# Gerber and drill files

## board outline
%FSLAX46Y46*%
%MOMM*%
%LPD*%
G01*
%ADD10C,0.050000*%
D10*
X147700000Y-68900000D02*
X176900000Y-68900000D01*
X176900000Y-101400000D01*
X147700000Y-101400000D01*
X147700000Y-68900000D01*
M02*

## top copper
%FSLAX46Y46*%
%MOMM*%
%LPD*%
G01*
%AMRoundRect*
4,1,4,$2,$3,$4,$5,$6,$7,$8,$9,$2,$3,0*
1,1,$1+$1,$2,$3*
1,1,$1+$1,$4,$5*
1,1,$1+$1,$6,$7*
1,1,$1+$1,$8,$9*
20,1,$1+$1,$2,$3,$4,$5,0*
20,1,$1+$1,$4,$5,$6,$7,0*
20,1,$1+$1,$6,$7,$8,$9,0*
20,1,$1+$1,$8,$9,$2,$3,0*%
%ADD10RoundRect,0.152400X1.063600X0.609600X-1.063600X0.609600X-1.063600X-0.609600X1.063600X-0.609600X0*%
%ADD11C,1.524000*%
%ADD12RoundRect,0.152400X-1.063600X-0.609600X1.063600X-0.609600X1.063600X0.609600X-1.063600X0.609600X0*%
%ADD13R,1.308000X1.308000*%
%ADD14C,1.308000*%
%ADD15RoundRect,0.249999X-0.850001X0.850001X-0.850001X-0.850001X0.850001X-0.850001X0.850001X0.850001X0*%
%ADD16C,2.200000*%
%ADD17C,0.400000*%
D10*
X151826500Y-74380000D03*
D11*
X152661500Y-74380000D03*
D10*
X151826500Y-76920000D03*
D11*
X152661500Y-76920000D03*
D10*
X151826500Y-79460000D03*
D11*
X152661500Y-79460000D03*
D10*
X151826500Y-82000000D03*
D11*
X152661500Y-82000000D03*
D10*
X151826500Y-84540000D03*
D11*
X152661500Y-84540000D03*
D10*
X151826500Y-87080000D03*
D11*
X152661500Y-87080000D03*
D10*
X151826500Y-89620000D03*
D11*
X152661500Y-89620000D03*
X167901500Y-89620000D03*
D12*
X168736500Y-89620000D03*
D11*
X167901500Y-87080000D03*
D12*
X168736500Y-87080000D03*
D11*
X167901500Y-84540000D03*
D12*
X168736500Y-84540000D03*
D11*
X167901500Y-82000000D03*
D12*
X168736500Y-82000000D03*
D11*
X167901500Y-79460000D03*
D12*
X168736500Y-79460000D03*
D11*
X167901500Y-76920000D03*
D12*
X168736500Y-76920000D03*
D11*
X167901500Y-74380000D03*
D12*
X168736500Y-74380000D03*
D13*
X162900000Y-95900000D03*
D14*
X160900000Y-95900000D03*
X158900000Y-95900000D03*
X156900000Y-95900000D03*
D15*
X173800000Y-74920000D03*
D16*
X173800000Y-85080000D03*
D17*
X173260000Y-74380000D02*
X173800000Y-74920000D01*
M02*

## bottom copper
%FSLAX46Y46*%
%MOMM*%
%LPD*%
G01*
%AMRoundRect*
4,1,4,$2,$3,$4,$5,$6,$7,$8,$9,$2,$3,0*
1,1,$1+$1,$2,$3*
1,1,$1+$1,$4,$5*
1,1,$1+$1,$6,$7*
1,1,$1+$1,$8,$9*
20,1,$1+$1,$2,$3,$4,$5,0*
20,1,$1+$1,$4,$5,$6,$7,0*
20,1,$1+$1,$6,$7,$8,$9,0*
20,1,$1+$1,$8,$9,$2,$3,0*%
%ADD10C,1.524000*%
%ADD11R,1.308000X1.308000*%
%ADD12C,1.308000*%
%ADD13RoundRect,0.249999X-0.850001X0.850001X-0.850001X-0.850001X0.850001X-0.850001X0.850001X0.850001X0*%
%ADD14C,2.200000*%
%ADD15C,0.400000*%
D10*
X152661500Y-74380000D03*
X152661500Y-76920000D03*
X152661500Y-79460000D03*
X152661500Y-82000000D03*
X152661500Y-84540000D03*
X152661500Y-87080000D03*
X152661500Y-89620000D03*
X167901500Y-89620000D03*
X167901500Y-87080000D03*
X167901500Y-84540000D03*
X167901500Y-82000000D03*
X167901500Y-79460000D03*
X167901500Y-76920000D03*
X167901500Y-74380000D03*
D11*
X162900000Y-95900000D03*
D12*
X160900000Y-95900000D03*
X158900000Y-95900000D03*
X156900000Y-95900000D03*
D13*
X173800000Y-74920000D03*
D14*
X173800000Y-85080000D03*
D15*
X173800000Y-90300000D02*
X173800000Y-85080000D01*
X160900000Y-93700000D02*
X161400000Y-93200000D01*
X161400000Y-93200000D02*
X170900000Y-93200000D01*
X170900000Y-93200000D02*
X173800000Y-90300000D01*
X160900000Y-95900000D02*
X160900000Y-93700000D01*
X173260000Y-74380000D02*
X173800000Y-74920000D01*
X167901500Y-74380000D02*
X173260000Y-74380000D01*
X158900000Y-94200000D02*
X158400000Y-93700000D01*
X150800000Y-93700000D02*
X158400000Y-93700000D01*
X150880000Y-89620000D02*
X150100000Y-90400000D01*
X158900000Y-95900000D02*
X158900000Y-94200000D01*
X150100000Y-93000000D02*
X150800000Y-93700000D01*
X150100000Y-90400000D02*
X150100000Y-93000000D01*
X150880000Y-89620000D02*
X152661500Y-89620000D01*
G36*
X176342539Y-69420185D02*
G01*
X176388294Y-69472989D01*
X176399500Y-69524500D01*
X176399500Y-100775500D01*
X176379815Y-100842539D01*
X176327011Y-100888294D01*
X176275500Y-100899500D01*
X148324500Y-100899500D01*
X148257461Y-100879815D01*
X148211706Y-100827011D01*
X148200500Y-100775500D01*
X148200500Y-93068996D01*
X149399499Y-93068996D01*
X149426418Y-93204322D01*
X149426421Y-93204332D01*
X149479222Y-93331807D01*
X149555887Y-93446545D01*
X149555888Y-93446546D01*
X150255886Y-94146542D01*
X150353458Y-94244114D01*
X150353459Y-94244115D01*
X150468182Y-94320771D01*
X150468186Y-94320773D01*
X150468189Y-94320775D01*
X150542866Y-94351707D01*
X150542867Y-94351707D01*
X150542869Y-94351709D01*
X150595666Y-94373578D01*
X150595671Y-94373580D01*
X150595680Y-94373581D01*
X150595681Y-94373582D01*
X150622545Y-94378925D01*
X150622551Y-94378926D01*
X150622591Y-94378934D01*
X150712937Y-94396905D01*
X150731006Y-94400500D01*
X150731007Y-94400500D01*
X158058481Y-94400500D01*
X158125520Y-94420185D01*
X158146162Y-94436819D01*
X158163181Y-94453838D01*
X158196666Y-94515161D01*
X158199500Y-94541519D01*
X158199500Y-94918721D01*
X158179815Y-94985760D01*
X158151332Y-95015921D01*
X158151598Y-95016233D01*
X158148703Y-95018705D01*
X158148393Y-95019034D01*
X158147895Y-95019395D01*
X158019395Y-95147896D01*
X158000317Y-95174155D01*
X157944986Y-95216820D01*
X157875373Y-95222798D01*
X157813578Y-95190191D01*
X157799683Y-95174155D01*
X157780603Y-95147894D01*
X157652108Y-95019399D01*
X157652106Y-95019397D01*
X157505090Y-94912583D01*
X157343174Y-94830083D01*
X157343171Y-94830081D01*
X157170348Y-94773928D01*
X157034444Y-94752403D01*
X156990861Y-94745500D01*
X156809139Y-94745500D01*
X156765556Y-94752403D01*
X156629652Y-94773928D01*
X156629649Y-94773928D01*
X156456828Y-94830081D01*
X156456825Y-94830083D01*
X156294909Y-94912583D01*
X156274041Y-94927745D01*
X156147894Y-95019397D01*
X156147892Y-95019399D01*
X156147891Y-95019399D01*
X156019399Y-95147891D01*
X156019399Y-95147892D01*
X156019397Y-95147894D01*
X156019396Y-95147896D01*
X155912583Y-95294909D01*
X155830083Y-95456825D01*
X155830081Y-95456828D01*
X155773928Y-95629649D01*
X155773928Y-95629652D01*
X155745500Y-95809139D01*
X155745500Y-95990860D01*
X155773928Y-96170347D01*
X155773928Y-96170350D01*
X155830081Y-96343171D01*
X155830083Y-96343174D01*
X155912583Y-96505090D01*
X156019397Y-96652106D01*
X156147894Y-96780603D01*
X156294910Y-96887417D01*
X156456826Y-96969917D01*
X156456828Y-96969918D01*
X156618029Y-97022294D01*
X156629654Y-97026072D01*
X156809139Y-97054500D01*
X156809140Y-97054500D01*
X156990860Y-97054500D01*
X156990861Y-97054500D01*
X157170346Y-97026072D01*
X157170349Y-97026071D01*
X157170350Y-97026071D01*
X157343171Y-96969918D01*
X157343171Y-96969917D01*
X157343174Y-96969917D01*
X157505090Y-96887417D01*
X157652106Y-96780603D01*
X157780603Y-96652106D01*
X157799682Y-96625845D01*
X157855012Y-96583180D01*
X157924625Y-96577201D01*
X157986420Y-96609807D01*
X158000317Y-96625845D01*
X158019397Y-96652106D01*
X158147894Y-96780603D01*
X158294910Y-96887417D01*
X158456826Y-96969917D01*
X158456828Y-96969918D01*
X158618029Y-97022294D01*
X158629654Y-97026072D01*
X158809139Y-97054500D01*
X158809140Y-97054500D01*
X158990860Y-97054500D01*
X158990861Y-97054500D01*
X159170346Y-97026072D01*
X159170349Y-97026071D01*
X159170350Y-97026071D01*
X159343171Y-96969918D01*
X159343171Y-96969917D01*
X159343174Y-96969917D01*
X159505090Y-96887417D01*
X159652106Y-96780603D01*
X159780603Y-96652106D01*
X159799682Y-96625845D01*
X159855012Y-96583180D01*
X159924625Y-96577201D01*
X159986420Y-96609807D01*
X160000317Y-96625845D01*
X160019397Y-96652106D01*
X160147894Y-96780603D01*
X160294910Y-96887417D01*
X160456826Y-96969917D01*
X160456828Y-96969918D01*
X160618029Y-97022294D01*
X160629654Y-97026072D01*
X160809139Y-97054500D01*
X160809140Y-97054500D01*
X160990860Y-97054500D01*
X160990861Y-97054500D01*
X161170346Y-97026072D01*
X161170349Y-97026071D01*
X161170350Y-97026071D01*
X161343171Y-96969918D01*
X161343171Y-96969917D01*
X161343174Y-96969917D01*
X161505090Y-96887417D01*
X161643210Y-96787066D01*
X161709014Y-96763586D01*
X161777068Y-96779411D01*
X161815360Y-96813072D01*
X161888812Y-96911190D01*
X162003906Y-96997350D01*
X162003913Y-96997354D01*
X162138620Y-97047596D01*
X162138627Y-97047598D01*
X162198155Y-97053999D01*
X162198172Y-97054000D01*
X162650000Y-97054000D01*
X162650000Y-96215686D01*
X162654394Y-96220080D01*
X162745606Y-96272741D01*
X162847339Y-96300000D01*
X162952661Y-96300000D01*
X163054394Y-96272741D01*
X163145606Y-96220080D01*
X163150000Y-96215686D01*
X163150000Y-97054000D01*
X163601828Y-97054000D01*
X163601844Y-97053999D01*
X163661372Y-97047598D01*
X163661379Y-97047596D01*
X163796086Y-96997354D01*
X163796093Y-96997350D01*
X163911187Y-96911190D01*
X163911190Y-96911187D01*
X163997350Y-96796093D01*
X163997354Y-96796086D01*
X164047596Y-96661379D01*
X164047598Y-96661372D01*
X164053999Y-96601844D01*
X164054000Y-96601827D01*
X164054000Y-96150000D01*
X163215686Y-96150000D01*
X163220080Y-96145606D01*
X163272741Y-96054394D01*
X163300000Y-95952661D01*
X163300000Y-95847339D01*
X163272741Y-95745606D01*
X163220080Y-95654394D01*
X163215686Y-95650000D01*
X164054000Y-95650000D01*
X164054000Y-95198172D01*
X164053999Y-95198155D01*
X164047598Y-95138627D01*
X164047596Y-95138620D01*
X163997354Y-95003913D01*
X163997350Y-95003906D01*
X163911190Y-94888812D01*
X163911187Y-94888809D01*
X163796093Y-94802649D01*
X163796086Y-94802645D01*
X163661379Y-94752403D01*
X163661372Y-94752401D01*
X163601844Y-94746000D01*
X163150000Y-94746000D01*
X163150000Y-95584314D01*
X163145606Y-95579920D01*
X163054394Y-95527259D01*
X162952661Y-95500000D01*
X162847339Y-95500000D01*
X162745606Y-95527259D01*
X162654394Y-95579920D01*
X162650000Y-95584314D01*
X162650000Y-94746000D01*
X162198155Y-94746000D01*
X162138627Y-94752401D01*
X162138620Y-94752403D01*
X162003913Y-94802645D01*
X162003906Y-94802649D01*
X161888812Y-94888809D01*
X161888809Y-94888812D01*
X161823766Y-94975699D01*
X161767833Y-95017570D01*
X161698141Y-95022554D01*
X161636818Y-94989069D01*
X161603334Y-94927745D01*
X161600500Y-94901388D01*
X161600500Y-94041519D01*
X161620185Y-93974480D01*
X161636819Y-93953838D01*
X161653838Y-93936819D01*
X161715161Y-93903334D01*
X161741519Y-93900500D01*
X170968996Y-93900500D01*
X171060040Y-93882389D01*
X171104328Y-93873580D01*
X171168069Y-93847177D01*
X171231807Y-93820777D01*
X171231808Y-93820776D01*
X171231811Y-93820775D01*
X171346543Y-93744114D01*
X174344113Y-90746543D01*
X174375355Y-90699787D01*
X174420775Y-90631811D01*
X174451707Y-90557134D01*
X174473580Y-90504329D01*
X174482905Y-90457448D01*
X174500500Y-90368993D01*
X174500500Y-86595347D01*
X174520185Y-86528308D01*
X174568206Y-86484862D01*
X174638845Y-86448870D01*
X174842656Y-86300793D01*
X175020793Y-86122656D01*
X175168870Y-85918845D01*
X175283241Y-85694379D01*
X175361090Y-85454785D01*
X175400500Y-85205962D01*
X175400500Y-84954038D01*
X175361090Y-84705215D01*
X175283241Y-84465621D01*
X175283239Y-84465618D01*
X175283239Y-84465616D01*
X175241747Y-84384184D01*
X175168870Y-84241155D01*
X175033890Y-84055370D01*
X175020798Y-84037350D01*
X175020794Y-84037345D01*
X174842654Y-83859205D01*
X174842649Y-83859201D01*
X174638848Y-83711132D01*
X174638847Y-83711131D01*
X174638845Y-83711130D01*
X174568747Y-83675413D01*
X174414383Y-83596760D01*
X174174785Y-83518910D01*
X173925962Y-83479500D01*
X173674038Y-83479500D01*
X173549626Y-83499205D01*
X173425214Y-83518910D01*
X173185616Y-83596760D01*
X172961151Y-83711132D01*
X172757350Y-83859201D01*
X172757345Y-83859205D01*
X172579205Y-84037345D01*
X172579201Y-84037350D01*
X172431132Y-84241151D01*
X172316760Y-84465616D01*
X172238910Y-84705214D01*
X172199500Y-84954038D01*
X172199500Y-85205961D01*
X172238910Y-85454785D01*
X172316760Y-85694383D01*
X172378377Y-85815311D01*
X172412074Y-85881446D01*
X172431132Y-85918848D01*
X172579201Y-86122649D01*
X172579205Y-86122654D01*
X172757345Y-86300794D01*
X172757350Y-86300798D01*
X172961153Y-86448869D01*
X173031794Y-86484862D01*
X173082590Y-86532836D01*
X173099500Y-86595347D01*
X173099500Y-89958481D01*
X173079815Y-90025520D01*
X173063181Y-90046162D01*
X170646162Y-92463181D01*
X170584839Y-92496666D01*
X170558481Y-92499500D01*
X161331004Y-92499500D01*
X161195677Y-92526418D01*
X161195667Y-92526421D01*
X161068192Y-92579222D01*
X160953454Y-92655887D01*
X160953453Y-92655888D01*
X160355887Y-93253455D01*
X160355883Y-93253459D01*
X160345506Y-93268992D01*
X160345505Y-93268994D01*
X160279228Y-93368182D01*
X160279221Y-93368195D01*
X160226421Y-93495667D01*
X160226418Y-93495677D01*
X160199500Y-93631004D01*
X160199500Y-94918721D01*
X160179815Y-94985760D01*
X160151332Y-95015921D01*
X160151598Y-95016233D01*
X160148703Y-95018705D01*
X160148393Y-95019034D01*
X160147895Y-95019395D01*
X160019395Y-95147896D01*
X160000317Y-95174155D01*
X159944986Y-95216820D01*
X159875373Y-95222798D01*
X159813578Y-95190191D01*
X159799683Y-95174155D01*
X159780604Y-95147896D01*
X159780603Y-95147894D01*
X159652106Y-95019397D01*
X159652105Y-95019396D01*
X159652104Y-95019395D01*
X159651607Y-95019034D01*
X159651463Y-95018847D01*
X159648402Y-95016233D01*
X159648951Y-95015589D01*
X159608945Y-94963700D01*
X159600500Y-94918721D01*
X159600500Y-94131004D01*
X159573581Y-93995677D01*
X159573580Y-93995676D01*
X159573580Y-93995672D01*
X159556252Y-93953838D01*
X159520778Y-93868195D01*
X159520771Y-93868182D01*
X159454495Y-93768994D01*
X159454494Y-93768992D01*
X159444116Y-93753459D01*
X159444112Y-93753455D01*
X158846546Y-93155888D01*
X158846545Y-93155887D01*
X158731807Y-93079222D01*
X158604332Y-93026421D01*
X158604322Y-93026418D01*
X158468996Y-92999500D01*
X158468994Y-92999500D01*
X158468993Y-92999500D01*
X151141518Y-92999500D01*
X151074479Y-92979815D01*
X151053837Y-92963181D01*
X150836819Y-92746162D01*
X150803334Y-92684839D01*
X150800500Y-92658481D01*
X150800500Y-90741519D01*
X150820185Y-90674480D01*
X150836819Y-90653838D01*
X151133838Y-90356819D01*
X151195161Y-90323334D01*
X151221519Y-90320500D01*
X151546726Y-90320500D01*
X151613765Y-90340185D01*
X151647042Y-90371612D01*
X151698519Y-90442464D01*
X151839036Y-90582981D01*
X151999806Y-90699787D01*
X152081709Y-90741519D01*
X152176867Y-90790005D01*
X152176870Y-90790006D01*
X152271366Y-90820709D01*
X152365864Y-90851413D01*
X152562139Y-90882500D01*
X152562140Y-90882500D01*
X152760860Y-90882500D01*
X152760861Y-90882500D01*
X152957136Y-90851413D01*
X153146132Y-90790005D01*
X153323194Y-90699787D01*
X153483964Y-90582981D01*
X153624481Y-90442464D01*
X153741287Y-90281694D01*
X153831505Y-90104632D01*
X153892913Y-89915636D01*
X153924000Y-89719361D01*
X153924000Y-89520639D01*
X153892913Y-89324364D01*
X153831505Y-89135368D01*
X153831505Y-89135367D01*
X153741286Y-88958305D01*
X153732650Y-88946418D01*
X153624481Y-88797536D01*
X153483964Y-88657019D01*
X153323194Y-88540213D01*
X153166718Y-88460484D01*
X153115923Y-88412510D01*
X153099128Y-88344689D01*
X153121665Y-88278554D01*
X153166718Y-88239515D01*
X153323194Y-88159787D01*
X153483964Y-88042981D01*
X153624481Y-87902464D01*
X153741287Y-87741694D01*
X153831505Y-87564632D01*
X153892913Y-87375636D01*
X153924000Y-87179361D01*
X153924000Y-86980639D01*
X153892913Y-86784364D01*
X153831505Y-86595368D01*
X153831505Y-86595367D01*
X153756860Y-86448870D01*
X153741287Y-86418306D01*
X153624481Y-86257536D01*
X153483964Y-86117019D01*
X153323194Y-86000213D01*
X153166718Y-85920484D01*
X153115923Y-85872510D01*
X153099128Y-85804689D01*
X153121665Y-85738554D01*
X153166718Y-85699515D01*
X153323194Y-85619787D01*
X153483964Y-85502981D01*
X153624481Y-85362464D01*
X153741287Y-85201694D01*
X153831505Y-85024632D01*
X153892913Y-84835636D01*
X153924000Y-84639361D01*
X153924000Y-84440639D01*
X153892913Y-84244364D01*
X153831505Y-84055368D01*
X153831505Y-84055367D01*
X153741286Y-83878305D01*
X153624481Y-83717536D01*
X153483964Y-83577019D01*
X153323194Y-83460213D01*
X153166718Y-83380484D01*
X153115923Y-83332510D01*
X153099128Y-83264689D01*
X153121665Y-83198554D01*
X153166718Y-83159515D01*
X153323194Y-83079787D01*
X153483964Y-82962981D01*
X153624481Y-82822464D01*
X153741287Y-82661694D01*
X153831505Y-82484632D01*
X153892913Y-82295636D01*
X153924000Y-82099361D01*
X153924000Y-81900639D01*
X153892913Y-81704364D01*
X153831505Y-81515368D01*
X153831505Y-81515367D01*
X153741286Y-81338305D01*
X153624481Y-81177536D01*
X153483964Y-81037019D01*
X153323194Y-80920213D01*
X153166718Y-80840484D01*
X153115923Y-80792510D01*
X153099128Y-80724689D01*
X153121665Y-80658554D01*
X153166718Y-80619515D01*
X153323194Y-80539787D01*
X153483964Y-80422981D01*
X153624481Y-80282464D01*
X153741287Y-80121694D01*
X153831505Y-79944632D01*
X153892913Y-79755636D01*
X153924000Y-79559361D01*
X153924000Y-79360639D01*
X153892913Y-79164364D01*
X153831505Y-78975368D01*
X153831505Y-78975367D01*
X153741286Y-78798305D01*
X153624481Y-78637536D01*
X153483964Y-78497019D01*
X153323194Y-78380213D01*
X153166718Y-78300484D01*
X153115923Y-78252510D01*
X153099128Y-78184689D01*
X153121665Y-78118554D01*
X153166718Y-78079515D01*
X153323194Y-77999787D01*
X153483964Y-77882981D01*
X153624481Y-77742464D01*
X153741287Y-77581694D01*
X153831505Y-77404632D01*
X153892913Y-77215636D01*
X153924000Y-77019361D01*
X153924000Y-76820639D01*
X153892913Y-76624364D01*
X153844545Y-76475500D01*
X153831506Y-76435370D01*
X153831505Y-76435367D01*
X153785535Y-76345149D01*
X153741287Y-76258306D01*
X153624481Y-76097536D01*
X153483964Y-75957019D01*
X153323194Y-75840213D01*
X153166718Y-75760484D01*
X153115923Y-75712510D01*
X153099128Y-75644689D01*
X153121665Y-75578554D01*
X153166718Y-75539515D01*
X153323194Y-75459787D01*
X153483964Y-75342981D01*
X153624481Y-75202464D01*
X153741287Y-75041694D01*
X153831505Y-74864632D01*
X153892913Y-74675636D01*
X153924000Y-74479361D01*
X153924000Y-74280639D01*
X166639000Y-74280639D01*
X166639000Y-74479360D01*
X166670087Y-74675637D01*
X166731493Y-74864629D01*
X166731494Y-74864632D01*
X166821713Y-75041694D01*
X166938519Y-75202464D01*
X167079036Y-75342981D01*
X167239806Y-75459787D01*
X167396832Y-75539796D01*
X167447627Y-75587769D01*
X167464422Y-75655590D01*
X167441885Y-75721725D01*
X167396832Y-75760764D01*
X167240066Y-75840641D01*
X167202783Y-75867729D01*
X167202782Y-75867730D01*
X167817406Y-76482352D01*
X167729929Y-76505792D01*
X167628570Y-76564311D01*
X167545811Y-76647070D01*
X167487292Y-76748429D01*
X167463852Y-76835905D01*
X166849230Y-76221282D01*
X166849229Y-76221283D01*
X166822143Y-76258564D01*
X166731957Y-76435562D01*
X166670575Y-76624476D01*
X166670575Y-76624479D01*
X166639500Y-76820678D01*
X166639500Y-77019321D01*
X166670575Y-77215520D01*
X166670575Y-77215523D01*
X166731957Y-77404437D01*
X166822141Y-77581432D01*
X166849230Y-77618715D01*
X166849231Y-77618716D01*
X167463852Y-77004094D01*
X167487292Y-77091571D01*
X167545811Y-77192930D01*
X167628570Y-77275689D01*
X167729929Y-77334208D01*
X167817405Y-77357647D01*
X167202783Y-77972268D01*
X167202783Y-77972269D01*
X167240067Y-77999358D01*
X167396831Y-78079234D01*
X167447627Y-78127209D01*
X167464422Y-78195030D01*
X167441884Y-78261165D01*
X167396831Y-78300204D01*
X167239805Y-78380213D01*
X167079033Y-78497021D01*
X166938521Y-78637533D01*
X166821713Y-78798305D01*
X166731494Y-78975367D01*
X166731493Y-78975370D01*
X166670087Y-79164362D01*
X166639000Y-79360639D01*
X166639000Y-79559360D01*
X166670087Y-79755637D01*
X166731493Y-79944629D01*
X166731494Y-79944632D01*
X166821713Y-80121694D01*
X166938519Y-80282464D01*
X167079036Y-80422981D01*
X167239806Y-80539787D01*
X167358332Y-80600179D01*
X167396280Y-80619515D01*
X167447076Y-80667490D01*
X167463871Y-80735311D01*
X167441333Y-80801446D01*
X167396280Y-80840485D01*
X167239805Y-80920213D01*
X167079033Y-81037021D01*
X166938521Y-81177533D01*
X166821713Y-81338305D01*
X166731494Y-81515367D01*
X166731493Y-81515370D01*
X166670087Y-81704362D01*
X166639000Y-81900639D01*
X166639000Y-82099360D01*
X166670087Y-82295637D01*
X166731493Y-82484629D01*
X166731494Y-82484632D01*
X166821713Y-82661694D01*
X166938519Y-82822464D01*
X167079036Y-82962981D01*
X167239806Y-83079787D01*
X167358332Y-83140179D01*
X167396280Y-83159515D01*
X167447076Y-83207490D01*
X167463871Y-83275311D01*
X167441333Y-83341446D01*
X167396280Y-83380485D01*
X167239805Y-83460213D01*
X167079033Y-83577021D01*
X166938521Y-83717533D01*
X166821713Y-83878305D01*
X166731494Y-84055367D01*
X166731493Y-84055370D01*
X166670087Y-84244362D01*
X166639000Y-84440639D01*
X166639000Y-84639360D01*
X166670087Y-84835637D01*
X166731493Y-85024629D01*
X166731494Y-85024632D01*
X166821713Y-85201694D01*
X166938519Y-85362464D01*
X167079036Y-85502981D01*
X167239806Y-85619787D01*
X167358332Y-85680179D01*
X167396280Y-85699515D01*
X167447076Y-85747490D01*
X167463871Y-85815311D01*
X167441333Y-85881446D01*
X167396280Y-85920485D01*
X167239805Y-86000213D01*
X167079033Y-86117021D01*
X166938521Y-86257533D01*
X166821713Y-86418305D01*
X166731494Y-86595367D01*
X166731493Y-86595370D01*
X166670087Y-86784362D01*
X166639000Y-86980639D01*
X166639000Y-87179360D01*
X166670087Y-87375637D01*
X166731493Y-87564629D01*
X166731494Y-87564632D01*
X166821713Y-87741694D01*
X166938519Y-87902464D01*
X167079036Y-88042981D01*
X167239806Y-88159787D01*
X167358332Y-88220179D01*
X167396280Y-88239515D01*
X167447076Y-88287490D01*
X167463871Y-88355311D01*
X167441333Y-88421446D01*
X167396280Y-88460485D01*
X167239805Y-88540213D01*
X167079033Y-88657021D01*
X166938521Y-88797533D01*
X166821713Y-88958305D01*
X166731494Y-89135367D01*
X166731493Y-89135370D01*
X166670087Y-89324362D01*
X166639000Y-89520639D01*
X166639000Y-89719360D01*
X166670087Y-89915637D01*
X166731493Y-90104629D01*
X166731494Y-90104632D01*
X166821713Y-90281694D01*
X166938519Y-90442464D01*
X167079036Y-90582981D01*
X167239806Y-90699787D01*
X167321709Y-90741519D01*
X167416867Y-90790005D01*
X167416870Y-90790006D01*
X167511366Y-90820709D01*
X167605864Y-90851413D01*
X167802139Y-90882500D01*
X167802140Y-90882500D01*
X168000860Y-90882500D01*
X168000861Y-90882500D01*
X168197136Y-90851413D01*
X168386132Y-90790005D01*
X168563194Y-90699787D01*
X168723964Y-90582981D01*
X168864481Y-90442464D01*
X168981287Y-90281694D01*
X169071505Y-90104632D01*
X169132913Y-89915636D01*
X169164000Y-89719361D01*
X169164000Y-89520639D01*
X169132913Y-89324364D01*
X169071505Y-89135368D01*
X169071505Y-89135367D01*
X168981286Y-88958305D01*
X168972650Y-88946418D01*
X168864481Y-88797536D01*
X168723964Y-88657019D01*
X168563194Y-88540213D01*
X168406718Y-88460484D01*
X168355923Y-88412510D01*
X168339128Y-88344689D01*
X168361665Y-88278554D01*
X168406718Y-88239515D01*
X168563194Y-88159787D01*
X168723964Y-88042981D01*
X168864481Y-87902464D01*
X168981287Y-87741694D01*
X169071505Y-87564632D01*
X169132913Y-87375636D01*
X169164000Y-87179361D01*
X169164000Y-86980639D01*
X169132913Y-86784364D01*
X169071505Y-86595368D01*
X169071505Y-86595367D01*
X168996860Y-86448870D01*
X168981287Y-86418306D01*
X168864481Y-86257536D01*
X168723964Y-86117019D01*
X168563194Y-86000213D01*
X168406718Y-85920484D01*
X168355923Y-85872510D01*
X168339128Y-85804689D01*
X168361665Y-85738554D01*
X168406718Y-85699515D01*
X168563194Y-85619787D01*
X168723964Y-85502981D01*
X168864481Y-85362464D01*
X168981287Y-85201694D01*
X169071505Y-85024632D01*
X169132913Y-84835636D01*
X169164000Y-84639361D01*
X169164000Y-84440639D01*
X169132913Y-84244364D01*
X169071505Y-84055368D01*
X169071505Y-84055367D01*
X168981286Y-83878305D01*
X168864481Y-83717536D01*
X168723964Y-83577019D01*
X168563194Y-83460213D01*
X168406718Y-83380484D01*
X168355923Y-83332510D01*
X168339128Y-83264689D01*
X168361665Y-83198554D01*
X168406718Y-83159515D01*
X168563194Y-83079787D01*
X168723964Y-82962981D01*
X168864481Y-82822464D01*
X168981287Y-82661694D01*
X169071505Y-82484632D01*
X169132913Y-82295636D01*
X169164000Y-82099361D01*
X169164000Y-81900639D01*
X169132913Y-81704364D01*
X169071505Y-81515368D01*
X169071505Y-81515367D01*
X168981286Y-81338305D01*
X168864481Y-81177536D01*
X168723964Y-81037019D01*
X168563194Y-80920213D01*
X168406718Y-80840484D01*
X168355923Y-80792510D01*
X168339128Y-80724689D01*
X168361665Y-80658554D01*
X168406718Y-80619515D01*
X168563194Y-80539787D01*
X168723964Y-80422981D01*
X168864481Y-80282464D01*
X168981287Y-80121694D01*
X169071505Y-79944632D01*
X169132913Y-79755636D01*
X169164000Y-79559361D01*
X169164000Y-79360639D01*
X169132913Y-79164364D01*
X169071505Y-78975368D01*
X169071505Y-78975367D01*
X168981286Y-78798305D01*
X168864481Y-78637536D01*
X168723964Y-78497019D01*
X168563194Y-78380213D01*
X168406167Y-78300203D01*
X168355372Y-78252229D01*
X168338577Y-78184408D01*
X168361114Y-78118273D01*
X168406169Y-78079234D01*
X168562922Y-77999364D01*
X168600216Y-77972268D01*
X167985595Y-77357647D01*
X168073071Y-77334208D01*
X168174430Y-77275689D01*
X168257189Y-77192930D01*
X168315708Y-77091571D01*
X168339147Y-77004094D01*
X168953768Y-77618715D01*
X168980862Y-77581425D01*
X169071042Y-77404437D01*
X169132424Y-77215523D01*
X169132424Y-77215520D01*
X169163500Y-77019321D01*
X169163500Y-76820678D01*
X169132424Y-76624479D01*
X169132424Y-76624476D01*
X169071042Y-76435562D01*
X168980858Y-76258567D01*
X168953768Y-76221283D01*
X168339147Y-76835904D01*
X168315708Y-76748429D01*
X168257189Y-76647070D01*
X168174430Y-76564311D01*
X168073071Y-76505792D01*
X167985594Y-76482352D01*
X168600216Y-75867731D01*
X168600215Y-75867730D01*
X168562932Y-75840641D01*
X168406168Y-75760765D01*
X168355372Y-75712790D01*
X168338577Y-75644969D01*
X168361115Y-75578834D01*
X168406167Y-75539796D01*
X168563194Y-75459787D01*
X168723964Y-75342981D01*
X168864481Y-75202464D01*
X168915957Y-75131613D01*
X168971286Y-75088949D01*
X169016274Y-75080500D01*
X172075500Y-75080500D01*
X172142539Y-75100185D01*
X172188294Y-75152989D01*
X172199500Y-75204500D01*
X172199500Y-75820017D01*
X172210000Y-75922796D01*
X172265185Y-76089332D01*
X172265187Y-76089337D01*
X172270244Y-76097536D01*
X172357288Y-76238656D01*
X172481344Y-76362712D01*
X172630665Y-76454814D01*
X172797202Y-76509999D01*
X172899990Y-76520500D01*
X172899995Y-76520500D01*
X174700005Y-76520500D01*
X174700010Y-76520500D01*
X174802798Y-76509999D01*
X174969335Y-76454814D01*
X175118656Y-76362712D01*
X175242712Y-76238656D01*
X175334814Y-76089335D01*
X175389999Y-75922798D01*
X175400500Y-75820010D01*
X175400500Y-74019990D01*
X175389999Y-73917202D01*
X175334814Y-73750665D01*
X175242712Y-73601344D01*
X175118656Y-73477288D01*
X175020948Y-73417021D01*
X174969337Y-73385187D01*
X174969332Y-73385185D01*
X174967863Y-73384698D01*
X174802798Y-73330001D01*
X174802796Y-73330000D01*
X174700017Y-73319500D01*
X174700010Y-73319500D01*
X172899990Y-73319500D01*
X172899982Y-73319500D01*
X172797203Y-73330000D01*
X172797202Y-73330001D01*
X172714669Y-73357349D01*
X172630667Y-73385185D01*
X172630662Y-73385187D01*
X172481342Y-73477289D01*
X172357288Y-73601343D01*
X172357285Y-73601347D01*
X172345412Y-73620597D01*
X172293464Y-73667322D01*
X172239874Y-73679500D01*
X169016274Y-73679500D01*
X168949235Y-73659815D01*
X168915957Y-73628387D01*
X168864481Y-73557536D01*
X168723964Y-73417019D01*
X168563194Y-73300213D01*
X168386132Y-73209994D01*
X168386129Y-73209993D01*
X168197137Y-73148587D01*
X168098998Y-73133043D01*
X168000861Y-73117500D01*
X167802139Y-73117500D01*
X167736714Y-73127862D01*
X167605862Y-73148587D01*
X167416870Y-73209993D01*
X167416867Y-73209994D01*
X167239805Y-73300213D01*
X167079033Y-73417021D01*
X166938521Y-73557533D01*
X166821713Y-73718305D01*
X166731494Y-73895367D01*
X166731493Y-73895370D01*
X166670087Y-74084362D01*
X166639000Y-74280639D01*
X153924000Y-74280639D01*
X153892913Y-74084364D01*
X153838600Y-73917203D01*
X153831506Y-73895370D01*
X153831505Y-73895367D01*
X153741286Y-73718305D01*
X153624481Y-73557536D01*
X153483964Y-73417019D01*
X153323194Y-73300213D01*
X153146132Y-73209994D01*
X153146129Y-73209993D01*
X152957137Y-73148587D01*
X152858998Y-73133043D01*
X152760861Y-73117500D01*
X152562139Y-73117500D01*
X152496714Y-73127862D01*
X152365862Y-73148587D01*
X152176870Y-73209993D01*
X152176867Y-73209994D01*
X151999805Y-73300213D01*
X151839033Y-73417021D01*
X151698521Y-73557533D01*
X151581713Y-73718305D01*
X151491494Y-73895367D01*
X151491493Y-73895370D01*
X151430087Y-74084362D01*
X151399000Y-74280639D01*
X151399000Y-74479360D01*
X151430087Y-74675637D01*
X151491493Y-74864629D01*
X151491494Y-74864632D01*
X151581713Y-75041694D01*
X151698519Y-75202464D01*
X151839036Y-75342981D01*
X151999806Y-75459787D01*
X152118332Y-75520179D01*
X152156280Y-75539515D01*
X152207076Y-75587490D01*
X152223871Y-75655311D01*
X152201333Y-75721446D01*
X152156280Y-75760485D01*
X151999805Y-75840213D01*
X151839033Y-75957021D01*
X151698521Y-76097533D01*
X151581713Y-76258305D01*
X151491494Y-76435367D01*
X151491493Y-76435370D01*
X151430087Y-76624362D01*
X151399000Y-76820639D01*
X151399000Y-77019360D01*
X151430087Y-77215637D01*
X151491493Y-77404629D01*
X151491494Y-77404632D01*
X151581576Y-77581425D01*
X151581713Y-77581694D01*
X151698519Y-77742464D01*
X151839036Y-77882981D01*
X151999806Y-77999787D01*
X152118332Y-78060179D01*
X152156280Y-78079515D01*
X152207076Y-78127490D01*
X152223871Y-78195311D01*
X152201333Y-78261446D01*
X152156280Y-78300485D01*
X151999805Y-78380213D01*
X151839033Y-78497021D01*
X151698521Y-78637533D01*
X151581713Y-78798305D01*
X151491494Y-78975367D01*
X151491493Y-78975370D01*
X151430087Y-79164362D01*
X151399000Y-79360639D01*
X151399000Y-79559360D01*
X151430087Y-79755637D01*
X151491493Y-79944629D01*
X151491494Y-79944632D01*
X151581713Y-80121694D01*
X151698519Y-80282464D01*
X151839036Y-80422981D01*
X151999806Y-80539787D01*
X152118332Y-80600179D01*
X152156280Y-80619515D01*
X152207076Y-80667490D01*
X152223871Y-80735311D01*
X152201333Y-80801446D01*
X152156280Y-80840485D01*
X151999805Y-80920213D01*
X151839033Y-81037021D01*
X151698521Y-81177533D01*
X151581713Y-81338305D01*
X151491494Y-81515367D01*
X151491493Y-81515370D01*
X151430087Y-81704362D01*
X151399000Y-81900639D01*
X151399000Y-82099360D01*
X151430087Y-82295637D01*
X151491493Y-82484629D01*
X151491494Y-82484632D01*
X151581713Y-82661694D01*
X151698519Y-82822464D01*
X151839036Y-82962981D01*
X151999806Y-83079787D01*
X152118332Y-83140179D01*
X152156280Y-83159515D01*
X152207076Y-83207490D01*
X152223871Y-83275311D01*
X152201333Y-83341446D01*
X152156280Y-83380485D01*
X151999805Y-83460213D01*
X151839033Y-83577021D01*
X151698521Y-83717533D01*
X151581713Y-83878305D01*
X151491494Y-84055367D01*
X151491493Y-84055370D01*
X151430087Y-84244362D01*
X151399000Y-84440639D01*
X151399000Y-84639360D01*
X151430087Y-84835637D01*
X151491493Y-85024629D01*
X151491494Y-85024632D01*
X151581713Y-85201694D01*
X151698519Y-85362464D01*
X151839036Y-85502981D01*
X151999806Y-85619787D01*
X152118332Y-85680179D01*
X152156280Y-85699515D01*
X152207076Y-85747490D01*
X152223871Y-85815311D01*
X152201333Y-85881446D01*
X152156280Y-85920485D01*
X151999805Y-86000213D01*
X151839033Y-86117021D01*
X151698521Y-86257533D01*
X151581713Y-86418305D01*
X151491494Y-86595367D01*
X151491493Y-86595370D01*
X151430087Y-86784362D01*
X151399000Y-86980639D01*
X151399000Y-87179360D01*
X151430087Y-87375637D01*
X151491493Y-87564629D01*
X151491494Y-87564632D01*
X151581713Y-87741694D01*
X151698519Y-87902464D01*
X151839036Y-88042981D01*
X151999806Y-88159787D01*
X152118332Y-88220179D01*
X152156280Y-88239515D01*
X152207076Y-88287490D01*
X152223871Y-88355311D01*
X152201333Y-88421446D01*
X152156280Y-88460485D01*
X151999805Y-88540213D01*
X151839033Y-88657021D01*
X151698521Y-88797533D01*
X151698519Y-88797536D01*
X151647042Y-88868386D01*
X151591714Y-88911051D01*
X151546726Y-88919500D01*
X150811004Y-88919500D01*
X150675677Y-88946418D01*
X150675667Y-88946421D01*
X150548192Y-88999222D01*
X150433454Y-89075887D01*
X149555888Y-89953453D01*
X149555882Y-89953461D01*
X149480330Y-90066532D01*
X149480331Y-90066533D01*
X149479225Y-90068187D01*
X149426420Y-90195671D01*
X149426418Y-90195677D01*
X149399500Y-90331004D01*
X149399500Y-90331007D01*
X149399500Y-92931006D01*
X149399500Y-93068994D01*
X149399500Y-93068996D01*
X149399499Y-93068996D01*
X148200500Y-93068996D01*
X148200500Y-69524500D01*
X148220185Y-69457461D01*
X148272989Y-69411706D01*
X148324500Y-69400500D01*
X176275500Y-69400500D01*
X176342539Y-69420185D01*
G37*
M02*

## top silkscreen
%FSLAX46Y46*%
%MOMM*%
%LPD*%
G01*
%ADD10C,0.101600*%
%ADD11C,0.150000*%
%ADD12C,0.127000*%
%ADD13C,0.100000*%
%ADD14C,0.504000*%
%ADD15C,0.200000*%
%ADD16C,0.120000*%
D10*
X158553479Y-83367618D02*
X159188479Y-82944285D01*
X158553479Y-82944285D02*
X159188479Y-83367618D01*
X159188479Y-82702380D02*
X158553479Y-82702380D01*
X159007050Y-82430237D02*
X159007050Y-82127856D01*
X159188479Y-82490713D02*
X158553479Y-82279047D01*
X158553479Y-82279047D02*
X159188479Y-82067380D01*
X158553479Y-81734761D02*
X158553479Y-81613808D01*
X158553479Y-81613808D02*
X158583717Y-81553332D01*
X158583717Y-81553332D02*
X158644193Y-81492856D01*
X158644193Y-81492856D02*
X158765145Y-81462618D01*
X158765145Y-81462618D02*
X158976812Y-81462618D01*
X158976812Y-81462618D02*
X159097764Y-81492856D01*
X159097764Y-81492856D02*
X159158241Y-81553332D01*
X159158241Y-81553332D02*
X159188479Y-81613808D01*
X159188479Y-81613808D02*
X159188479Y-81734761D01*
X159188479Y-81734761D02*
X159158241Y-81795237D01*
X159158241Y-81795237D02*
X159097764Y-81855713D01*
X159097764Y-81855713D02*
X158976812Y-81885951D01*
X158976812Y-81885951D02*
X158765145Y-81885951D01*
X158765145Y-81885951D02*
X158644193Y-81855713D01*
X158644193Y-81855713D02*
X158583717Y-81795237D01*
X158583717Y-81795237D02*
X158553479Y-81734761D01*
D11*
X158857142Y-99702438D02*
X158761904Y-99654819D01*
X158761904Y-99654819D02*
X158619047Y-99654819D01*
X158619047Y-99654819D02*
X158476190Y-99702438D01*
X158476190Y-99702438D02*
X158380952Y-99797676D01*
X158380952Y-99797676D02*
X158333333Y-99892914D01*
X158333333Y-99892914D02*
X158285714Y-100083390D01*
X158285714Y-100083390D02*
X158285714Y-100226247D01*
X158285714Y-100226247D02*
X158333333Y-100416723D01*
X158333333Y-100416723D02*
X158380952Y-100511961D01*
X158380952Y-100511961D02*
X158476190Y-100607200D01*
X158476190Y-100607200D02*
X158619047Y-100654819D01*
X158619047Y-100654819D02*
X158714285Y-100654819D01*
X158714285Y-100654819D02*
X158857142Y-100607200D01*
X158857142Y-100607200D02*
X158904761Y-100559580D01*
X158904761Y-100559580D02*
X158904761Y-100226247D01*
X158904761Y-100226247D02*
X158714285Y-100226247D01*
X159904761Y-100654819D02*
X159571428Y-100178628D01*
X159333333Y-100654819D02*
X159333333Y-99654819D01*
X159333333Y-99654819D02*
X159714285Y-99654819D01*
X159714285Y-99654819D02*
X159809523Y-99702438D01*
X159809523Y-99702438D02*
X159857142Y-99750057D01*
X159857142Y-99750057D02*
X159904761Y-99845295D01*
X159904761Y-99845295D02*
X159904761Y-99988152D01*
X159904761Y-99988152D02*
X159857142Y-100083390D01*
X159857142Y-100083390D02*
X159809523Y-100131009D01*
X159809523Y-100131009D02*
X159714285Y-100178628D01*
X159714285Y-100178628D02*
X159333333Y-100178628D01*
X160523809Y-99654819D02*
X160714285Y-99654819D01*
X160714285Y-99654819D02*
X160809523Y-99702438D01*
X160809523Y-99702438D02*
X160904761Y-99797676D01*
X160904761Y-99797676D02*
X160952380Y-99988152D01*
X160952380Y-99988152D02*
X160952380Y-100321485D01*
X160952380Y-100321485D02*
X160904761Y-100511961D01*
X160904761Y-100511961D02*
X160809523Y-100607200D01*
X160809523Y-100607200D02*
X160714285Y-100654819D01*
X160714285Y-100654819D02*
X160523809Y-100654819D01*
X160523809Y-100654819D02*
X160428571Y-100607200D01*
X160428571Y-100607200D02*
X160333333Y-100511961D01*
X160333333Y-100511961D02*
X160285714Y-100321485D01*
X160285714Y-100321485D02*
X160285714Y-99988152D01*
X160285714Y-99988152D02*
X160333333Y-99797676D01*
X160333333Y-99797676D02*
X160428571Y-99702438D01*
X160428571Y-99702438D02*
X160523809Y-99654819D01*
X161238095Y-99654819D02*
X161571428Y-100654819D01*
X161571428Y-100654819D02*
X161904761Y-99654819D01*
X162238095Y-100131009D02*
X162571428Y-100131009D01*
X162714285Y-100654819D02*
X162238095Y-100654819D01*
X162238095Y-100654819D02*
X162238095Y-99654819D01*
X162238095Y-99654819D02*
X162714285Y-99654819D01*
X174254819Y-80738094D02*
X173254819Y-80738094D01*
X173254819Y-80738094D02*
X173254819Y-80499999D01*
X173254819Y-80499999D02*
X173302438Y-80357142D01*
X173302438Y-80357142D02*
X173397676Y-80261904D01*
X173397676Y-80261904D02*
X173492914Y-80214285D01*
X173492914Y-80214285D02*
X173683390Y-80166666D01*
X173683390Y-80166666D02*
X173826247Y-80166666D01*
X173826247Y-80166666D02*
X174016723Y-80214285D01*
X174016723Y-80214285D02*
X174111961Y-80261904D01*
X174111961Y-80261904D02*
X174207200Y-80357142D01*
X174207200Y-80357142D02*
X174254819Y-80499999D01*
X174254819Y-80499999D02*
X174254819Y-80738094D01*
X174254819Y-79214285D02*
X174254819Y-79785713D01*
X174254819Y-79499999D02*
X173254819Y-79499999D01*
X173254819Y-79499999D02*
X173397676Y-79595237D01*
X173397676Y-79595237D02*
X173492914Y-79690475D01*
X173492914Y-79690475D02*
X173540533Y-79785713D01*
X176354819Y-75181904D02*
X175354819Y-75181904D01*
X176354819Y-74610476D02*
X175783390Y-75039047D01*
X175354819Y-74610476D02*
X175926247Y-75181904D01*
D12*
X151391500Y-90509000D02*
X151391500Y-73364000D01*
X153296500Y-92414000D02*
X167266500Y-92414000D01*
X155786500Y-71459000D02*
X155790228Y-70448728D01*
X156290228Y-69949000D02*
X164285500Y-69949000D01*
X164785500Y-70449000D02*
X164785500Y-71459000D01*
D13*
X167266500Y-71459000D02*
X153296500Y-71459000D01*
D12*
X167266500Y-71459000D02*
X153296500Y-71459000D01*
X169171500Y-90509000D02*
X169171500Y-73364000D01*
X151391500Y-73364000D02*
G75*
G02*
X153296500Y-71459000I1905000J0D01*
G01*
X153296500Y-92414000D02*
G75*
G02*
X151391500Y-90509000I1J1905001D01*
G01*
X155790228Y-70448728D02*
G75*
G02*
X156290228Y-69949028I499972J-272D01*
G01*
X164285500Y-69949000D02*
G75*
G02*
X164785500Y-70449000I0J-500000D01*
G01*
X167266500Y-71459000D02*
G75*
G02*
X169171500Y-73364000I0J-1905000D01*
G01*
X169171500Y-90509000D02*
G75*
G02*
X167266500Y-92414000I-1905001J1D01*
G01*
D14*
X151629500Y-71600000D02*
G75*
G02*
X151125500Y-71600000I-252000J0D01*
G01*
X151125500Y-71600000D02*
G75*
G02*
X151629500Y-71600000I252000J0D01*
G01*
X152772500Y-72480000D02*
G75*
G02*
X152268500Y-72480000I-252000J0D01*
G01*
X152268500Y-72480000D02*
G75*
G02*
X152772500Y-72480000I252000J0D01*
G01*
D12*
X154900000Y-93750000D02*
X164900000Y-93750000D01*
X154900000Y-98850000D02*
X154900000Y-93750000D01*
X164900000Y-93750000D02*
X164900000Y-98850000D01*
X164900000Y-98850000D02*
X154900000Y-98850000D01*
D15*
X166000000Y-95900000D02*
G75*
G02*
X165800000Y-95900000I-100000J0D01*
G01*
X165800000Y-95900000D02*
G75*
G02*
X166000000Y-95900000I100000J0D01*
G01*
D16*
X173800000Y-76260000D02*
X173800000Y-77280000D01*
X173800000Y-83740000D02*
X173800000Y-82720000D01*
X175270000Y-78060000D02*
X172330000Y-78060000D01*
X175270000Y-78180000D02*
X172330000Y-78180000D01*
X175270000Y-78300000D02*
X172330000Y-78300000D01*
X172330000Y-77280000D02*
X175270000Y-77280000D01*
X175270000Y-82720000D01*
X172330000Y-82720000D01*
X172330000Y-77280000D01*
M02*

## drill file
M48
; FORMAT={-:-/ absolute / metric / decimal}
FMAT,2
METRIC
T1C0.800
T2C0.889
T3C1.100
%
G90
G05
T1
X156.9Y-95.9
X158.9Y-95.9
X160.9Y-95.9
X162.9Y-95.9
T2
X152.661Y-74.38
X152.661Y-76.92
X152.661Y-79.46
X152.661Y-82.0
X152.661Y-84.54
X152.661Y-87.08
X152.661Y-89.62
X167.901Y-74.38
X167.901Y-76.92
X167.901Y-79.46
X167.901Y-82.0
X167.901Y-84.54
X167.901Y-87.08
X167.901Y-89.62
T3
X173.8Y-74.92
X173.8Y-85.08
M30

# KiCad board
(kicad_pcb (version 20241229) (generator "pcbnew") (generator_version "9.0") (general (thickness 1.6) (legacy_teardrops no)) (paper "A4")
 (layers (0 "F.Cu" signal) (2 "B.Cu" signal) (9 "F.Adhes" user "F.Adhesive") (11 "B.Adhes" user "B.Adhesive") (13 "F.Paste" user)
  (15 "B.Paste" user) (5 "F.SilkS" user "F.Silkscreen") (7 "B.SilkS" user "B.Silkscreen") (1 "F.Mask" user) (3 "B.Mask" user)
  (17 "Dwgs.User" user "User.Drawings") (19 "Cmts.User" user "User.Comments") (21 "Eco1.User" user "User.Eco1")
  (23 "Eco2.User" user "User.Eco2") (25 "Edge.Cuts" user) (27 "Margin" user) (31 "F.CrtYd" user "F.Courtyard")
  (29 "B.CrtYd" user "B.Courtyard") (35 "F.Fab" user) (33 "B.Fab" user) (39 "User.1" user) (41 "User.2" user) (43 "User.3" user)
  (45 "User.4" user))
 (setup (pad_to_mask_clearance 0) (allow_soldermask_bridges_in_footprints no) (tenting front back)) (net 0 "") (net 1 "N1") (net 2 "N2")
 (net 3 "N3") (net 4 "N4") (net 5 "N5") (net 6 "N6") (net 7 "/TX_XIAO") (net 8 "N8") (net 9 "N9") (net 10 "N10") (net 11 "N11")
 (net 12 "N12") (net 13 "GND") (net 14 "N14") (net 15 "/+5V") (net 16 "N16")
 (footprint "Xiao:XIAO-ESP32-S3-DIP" (layer "F.Cu") (at 160.2815 82 90)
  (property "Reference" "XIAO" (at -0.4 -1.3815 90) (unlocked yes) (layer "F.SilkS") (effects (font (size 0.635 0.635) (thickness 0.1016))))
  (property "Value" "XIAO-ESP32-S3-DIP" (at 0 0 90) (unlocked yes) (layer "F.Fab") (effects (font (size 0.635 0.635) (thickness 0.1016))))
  (fp_line (start -8.509 -8.89) (end 8.636 -8.89) (stroke (width 0.127) (type solid)) (layer "F.SilkS"))
  (fp_line (start -10.414 -6.985) (end -10.414 6.985) (stroke (width 0.127) (type solid)) (layer "F.SilkS"))
  (fp_line (start 10.541 -4.495) (end 11.551272 -4.491272) (stroke (width 0.127) (type solid)) (layer "F.SilkS"))
  (fp_line (start 12.051 -3.991272) (end 12.051 4.004) (stroke (width 0.127) (type solid)) (layer "F.SilkS"))
  (fp_line (start 11.551 4.504) (end 10.541 4.504) (stroke (width 0.127) (type solid)) (layer "F.SilkS"))
  (fp_line (start 10.541 6.985) (end 10.541 -6.985) (stroke (width 0.1) (type solid)) (layer "F.SilkS"))
  (fp_line (start 10.541 6.985) (end 10.541 -6.985) (stroke (width 0.127) (type solid)) (layer "F.SilkS"))
  (fp_line (start -8.509 8.89) (end 8.636 8.89) (stroke (width 0.127) (type solid)) (layer "F.SilkS"))
  (fp_arc (start 8.636 -8.89) (mid 9.983038 -8.332038) (end 10.541 -6.985) (stroke (width 0.127) (type solid)) (layer "F.SilkS"))
  (fp_arc (start -10.414 -6.985) (mid -9.856038 -8.332038) (end -8.509 -8.89) (stroke (width 0.127) (type solid)) (layer "F.SilkS"))
  (fp_arc (start 11.551272 -4.491272) (mid 11.904644 -4.344724) (end 12.051 -3.991272) (stroke (width 0.127) (type default))
   (layer "F.SilkS"))
  (fp_arc (start 12.051 4.004) (mid 11.904553 4.357553) (end 11.551 4.504) (stroke (width 0.127) (type default)) (layer "F.SilkS"))
  (fp_arc (start 10.541 6.985) (mid 9.983038 8.332038) (end 8.636 8.89) (stroke (width 0.127) (type solid)) (layer "F.SilkS"))
  (fp_arc (start -8.509 8.89) (mid -9.856038 8.332038) (end -10.414 6.985) (stroke (width 0.127) (type solid)) (layer "F.SilkS"))
  (fp_circle (center 10.4 -8.904) (end 10.654 -8.904) (stroke (width 0.5) (type solid)) (fill yes) (layer "F.SilkS"))
  (fp_circle (center 9.52 -7.761) (end 9.774 -7.761) (stroke (width 0.5) (type solid)) (fill yes) (layer "F.SilkS"))
  (pad "1" smd roundrect (at 7.62 -8.455 180) (size 2.432 1.524) (layers "F.Cu" "F.Mask") (roundrect_rratio 0.1) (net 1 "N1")
   (thermal_bridge_angle 45))
  (pad "1" thru_hole circle (at 7.62 -7.62 180) (size 1.524 1.524) (drill 0.889) (layers "*.Cu" "*.Mask") (remove_unused_layers no)
   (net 1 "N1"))
  (pad "2" smd roundrect (at 5.08 -8.455 180) (size 2.432 1.524) (layers "F.Cu" "F.Mask") (roundrect_rratio 0.1) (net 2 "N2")
   (thermal_bridge_angle 45))
  (pad "2" thru_hole circle (at 5.08 -7.62 180) (size 1.524 1.524) (drill 0.889) (layers "*.Cu" "*.Mask") (remove_unused_layers no)
   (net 2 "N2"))
  (pad "3" smd roundrect (at 2.54 -8.455 180) (size 2.432 1.524) (layers "F.Cu" "F.Mask") (roundrect_rratio 0.1) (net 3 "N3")
   (thermal_bridge_angle 45))
  (pad "3" thru_hole circle (at 2.54 -7.62 180) (size 1.524 1.524) (drill 0.889) (layers "*.Cu" "*.Mask") (remove_unused_layers no)
   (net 3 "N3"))
  (pad "4" smd roundrect (at 0 -8.455 180) (size 2.432 1.524) (layers "F.Cu" "F.Mask") (roundrect_rratio 0.1) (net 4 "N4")
   (thermal_bridge_angle 45))
  (pad "4" thru_hole circle (at 0 -7.62 180) (size 1.524 1.524) (drill 0.889) (layers "*.Cu" "*.Mask") (remove_unused_layers no)
   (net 4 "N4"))
  (pad "5" smd roundrect (at -2.54 -8.455 180) (size 2.432 1.524) (layers "F.Cu" "F.Mask") (roundrect_rratio 0.1) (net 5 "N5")
   (thermal_bridge_angle 45))
  (pad "5" thru_hole circle (at -2.54 -7.62 180) (size 1.524 1.524) (drill 0.889) (layers "*.Cu" "*.Mask") (remove_unused_layers no)
   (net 5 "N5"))
  (pad "6" smd roundrect (at -5.08 -8.455 180) (size 2.432 1.524) (layers "F.Cu" "F.Mask") (roundrect_rratio 0.1) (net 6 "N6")
   (thermal_bridge_angle 45))
  (pad "6" thru_hole circle (at -5.08 -7.62 180) (size 1.524 1.524) (drill 0.889) (layers "*.Cu" "*.Mask") (remove_unused_layers no)
   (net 6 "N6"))
  (pad "7" smd roundrect (at -7.62 -8.455 180) (size 2.432 1.524) (layers "F.Cu" "F.Mask") (roundrect_rratio 0.1) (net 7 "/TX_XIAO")
   (thermal_bridge_angle 45))
  (pad "7" thru_hole circle (at -7.62 -7.62 180) (size 1.524 1.524) (drill 0.889) (layers "*.Cu" "*.Mask") (remove_unused_layers no)
   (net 7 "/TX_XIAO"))
  (pad "8" thru_hole circle (at -7.62 7.62) (size 1.524 1.524) (drill 0.889) (layers "*.Cu" "*.Mask") (remove_unused_layers no) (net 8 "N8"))
  (pad "8" smd roundrect (at -7.62 8.455) (size 2.432 1.524) (layers "F.Cu" "F.Mask") (roundrect_rratio 0.1) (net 8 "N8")
   (thermal_bridge_angle 45))
  (pad "9" thru_hole circle (at -5.08 7.62) (size 1.524 1.524) (drill 0.889) (layers "*.Cu" "*.Mask") (remove_unused_layers no) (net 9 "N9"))
  (pad "9" smd roundrect (at -5.08 8.455) (size 2.432 1.524) (layers "F.Cu" "F.Mask") (roundrect_rratio 0.1) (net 9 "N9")
   (thermal_bridge_angle 45))
  (pad "10" thru_hole circle (at -2.54 7.62) (size 1.524 1.524) (drill 0.889) (layers "*.Cu" "*.Mask") (remove_unused_layers no)
   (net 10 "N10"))
  (pad "10" smd roundrect (at -2.54 8.455) (size 2.432 1.524) (layers "F.Cu" "F.Mask") (roundrect_rratio 0.1) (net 10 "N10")
   (thermal_bridge_angle 45))
  (pad "11" thru_hole circle (at 0 7.62) (size 1.524 1.524) (drill 0.889) (layers "*.Cu" "*.Mask") (remove_unused_layers no) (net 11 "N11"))
  (pad "11" smd roundrect (at 0 8.455) (size 2.432 1.524) (layers "F.Cu" "F.Mask") (roundrect_rratio 0.1) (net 11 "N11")
   (thermal_bridge_angle 45))
  (pad "12" thru_hole circle (at 2.54 7.62) (size 1.524 1.524) (drill 0.889) (layers "*.Cu" "*.Mask") (remove_unused_layers no)
   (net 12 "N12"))
  (pad "12" smd roundrect (at 2.54 8.455) (size 2.432 1.524) (layers "F.Cu" "F.Mask") (roundrect_rratio 0.1) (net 12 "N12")
   (thermal_bridge_angle 45))
  (pad "13" thru_hole circle (at 5.08 7.62) (size 1.524 1.524) (drill 0.889) (layers "*.Cu" "*.Mask") (remove_unused_layers no)
   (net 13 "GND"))
  (pad "13" smd roundrect (at 5.08 8.455) (size 2.432 1.524) (layers "F.Cu" "F.Mask") (roundrect_rratio 0.1) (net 13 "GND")
   (thermal_bridge_angle 45))
  (pad "14" thru_hole circle (at 7.62 7.62) (size 1.524 1.524) (drill 0.889) (layers "*.Cu" "*.Mask") (remove_unused_layers no)
   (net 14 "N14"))
  (pad "14" smd roundrect (at 7.62 8.455) (size 2.432 1.524) (layers "F.Cu" "F.Mask") (roundrect_rratio 0.1) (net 14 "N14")
   (thermal_bridge_angle 45)))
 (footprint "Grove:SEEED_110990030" (layer "F.Cu") (at 159.9 95.9)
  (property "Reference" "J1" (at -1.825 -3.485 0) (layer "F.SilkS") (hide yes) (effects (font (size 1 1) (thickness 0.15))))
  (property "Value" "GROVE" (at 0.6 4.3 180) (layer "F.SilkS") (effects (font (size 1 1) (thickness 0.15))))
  (fp_line (start -5 -2.15) (end 5 -2.15) (stroke (width 0.127) (type solid)) (layer "F.SilkS"))
  (fp_line (start -5 2.95) (end -5 -2.15) (stroke (width 0.127) (type solid)) (layer "F.SilkS"))
  (fp_line (start 5 -2.15) (end 5 2.95) (stroke (width 0.127) (type solid)) (layer "F.SilkS"))
  (fp_line (start 5 2.95) (end -5 2.95) (stroke (width 0.127) (type solid)) (layer "F.SilkS"))
  (fp_circle (center 6 0) (end 6.1 0) (stroke (width 0.2) (type solid)) (fill no) (layer "F.SilkS"))
  (pad "1" thru_hole rect (at 3 0) (size 1.308 1.308) (drill 0.8) (layers "*.Cu" "*.Mask") (remove_unused_layers no) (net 13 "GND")
   (solder_mask_margin 0.102))
  (pad "2" thru_hole circle (at 1 0) (size 1.308 1.308) (drill 0.8) (layers "*.Cu" "*.Mask") (remove_unused_layers no) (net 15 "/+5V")
   (solder_mask_margin 0.102))
  (pad "3" thru_hole circle (at -1 0) (size 1.308 1.308) (drill 0.8) (layers "*.Cu" "*.Mask") (remove_unused_layers no) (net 7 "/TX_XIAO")
   (solder_mask_margin 0.102))
  (pad "4" thru_hole circle (at -3 0) (size 1.308 1.308) (drill 0.8) (layers "*.Cu" "*.Mask") (remove_unused_layers no) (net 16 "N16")
   (solder_mask_margin 0.102)))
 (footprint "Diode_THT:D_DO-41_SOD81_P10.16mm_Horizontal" (layer "F.Cu") (at 173.8 74.92 -90)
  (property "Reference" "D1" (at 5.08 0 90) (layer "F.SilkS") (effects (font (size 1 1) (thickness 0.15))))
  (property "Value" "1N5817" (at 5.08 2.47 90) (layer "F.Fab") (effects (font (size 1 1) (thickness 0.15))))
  (fp_line (start 1.34 0) (end 2.36 0) (stroke (width 0.12) (type solid)) (layer "F.SilkS"))
  (fp_line (start 8.82 0) (end 7.8 0) (stroke (width 0.12) (type solid)) (layer "F.SilkS"))
  (fp_line (start 3.14 -1.47) (end 3.14 1.47) (stroke (width 0.12) (type solid)) (layer "F.SilkS"))
  (fp_line (start 3.26 -1.47) (end 3.26 1.47) (stroke (width 0.12) (type solid)) (layer "F.SilkS"))
  (fp_line (start 3.38 -1.47) (end 3.38 1.47) (stroke (width 0.12) (type solid)) (layer "F.SilkS"))
  (fp_rect (start 2.36 -1.47) (end 7.8 1.47) (stroke (width 0.12) (type solid)) (fill no) (layer "F.SilkS"))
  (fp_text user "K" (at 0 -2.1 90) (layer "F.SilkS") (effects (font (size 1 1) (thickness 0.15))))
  (pad "1" thru_hole roundrect (at 0 0 270) (size 2.2 2.2) (drill 1.1) (layers "*.Cu" "*.Mask") (remove_unused_layers no)
   (roundrect_rratio 0.113636) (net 14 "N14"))
  (pad "2" thru_hole circle (at 10.16 0 270) (size 2.2 2.2) (drill 1.1) (layers "*.Cu" "*.Mask") (remove_unused_layers no) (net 15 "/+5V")))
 (gr_rect (start 147.7 68.9) (end 176.9 101.4) (stroke (width 0.05) (type default)) (fill no) (layer "Edge.Cuts"))
 (segment (start 173.8 90.3) (end 173.8 85.08) (width 0.4) (layer "B.Cu") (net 15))
 (segment (start 160.9 93.7) (end 161.4 93.2) (width 0.4) (layer "B.Cu") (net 15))
 (segment (start 161.4 93.2) (end 170.9 93.2) (width 0.4) (layer "B.Cu") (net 15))
 (segment (start 170.9 93.2) (end 173.8 90.3) (width 0.4) (layer "B.Cu") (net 15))
 (segment (start 160.9 95.9) (end 160.9 93.7) (width 0.4) (layer "B.Cu") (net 15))
 (segment (start 173.26 74.38) (end 173.8 74.92) (width 0.4) (layer "F.Cu") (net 14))
 (segment (start 173.26 74.38) (end 173.8 74.92) (width 0.4) (layer "B.Cu") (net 14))
 (segment (start 167.9015 74.38) (end 173.26 74.38) (width 0.4) (layer "B.Cu") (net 14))
 (segment (start 158.9 94.2) (end 158.4 93.7) (width 0.4) (layer "B.Cu") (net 7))
 (segment (start 150.8 93.7) (end 158.4 93.7) (width 0.4) (layer "B.Cu") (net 7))
 (segment (start 150.88 89.62) (end 150.1 90.4) (width 0.4) (layer "B.Cu") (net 7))
 (segment (start 158.9 95.9) (end 158.9 94.2) (width 0.4) (layer "B.Cu") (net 7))
 (segment (start 150.1 93) (end 150.8 93.7) (width 0.4) (layer "B.Cu") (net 7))
 (segment (start 150.1 90.4) (end 150.1 93) (width 0.4) (layer "B.Cu") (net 7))
 (segment (start 150.88 89.62) (end 152.6615 89.62) (width 0.4) (layer "B.Cu") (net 7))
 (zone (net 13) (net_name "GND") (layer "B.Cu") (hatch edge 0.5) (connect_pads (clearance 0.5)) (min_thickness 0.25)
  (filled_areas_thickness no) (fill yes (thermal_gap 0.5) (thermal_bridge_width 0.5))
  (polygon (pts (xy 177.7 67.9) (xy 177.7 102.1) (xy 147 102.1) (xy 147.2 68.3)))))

